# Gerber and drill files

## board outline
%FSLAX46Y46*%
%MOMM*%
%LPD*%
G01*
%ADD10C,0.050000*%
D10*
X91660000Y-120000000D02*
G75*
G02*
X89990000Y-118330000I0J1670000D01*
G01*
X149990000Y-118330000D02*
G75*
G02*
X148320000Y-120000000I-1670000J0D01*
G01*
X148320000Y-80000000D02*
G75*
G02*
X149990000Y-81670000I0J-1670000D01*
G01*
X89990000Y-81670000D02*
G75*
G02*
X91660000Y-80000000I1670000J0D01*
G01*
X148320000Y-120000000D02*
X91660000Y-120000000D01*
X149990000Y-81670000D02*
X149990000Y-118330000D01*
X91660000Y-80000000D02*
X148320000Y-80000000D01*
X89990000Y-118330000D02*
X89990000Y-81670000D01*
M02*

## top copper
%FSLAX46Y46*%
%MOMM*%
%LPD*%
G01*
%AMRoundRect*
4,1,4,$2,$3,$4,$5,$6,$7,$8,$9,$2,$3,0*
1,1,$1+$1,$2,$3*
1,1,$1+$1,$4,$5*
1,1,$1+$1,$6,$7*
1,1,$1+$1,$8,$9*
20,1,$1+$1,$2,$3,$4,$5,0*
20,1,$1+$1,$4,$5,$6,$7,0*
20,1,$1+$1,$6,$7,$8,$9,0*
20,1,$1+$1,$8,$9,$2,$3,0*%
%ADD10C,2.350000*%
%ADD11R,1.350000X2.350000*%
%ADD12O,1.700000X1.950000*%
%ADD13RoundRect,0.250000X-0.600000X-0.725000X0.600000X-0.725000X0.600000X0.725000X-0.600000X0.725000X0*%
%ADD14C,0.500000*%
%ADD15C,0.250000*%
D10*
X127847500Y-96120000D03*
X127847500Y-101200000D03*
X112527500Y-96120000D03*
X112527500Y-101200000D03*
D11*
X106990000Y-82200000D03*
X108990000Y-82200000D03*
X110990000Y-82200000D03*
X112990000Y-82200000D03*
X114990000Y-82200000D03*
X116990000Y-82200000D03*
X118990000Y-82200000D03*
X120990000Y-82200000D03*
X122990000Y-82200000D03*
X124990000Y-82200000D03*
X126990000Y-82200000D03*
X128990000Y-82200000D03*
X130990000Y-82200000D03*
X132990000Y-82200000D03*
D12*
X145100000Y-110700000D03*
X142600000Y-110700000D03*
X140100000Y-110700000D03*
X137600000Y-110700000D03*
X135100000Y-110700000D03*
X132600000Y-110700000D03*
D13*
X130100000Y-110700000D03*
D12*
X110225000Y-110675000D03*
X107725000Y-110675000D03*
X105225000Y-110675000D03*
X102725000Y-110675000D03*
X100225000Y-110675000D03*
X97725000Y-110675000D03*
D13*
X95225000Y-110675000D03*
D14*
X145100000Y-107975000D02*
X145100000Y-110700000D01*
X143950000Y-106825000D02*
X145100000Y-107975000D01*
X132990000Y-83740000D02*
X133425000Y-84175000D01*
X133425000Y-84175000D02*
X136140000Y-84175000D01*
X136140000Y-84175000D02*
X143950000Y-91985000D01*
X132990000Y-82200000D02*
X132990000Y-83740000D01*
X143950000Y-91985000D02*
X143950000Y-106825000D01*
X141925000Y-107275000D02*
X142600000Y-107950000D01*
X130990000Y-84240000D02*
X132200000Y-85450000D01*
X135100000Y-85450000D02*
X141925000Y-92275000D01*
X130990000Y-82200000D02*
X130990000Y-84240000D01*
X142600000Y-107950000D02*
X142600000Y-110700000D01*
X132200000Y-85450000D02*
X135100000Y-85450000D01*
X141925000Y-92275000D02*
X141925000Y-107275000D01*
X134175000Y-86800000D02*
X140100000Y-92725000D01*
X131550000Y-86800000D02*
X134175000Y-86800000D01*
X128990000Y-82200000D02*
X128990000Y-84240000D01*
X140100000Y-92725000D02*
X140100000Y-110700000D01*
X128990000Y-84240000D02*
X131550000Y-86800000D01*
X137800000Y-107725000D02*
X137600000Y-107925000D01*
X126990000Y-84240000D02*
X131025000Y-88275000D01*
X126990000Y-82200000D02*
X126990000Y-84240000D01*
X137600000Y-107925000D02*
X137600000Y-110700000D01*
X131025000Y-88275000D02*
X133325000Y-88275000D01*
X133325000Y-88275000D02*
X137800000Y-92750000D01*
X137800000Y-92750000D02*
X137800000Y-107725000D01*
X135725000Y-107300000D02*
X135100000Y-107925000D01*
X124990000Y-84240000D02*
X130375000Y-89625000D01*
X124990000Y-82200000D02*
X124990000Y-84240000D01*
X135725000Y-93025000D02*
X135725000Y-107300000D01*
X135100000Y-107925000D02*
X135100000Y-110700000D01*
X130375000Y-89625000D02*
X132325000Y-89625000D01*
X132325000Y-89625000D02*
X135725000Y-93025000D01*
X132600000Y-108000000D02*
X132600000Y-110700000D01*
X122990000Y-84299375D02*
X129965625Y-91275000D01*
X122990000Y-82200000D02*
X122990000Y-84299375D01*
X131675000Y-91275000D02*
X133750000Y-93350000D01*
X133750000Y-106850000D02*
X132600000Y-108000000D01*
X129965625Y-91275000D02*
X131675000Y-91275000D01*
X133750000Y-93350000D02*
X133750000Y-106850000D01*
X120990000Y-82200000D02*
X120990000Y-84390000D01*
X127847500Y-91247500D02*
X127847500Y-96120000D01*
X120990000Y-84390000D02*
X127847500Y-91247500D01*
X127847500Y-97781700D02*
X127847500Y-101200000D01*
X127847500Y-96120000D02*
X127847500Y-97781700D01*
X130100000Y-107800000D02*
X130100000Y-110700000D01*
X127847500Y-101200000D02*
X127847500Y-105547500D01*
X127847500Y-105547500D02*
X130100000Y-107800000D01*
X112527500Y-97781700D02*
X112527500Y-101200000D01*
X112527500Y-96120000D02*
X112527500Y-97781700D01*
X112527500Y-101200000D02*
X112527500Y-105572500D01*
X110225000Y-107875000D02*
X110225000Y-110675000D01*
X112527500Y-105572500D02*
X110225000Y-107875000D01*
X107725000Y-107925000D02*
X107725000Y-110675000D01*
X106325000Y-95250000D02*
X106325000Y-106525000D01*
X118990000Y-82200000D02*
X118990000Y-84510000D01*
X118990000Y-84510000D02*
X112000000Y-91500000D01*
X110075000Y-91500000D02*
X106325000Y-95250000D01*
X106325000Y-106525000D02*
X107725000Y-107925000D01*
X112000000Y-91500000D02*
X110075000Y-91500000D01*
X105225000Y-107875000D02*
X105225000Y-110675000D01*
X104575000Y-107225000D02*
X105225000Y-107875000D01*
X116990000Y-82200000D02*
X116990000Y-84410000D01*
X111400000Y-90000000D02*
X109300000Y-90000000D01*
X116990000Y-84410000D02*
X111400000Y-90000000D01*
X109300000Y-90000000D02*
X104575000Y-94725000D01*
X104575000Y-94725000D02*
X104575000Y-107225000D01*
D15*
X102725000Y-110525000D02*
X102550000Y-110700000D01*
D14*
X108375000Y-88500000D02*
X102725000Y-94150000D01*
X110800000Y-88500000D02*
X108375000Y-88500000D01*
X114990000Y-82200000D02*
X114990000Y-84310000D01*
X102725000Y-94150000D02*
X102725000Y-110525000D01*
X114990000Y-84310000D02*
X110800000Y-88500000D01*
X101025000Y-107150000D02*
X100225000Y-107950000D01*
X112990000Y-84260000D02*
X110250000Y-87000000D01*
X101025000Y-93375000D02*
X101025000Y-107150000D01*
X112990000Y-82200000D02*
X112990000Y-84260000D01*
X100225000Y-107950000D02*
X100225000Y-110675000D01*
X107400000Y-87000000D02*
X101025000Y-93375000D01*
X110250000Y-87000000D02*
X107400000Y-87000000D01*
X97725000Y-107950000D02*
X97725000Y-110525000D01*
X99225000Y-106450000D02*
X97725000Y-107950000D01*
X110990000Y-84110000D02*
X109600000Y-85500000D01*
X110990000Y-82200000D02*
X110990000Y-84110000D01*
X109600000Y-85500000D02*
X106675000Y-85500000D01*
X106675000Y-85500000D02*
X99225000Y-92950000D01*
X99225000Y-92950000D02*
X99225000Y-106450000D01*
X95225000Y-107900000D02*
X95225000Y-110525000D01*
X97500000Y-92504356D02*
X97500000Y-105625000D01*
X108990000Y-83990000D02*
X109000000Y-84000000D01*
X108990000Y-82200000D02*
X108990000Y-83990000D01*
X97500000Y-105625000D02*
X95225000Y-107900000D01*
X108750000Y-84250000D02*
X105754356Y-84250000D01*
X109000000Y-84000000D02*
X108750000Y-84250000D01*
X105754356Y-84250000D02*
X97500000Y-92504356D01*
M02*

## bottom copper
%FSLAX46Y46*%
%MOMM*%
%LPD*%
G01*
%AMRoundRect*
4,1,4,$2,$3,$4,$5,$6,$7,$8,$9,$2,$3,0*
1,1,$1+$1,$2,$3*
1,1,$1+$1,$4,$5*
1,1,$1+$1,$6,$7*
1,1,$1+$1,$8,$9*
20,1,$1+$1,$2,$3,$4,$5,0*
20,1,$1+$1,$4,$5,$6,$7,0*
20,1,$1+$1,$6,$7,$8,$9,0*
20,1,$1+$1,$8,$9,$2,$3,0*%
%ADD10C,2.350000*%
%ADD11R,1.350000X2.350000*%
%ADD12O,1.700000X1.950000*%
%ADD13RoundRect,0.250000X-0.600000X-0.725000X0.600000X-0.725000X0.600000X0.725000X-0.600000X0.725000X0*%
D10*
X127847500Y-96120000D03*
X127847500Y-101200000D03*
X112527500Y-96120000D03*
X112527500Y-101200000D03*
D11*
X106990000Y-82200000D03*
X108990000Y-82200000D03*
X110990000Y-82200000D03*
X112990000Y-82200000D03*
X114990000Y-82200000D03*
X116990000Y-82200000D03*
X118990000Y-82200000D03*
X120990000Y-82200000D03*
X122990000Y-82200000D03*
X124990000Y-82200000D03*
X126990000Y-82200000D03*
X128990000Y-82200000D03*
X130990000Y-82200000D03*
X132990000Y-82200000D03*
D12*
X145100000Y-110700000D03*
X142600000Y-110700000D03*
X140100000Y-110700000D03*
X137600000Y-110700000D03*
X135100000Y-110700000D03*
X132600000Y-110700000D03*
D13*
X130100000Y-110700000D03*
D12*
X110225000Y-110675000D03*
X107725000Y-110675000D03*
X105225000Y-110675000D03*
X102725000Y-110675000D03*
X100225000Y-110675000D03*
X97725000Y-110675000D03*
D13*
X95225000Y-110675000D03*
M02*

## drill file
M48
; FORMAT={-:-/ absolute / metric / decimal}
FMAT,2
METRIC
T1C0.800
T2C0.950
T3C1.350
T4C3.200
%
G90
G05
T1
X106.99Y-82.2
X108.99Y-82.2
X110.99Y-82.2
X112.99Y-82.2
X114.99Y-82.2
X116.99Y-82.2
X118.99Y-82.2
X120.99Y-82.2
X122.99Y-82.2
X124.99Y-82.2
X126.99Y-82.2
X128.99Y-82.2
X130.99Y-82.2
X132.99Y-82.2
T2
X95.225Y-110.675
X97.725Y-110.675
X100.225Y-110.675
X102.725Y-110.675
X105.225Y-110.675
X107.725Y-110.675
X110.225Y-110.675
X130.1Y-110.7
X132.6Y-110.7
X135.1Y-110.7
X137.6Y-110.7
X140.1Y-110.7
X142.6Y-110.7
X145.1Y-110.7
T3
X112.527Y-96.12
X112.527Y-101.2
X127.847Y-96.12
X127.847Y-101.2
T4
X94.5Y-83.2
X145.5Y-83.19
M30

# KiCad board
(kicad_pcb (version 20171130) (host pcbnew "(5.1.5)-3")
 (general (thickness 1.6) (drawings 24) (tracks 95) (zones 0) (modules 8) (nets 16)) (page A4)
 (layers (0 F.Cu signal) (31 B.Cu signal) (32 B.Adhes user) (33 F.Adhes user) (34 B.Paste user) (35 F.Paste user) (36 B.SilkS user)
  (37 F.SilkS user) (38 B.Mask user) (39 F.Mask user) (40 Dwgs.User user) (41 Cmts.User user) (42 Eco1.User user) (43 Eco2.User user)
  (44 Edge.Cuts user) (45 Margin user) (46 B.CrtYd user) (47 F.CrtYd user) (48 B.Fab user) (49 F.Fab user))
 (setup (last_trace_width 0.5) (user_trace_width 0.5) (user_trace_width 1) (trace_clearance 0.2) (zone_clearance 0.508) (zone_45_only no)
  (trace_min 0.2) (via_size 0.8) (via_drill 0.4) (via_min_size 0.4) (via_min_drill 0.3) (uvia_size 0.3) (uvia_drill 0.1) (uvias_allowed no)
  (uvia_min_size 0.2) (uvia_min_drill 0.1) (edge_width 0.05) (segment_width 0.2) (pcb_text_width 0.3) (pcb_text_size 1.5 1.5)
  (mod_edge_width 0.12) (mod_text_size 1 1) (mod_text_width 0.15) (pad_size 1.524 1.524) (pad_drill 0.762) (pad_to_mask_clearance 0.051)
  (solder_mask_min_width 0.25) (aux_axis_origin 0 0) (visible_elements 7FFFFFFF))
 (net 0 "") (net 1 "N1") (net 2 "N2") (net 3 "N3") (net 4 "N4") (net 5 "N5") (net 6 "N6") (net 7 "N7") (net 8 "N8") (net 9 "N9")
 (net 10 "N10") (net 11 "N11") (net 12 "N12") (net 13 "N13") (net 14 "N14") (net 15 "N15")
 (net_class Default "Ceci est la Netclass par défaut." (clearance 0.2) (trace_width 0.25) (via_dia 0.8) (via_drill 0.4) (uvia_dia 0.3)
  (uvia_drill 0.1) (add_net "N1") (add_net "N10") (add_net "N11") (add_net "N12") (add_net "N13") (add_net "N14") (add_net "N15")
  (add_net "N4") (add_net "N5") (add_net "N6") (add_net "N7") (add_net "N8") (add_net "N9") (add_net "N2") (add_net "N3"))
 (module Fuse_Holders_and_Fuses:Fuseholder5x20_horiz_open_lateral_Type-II (layer F.Cu) (at 127.8475 101.2 180)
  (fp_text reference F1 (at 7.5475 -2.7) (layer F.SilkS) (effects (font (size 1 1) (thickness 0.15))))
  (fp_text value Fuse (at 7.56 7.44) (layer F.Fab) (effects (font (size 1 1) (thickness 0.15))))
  (pad 1 thru_hole circle (at 0 5.08 180) (size 2.35 2.35) (drill 1.35) (layers *.Cu *.Mask) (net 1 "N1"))
  (pad 1 thru_hole circle (at 0 0 180) (size 2.35 2.35) (drill 1.35) (layers *.Cu *.Mask) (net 1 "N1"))
  (pad 2 thru_hole circle (at 15.32 5.08 180) (size 2.35 2.35) (drill 1.35) (layers *.Cu *.Mask) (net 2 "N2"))
  (pad 2 thru_hole circle (at 15.32 0 180) (size 2.35 2.35) (drill 1.35) (layers *.Cu *.Mask) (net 2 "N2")))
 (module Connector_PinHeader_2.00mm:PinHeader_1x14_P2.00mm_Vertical (layer B.Cu) (at 132.99 82.2 90)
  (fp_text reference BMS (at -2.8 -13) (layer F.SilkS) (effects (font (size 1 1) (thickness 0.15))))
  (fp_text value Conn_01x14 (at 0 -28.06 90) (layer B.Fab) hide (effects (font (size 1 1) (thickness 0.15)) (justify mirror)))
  (pad 14 thru_hole rect (at 0 -26 90) (size 2.35 1.35) (drill 0.8) (layers *.Cu *.Mask) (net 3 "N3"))
  (pad 13 thru_hole rect (at 0 -24 90) (size 2.35 1.35) (drill 0.8) (layers *.Cu *.Mask) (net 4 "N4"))
  (pad 12 thru_hole rect (at 0 -22 90) (size 2.35 1.35) (drill 0.8) (layers *.Cu *.Mask) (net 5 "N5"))
  (pad 11 thru_hole rect (at 0 -20 90) (size 2.35 1.35) (drill 0.8) (layers *.Cu *.Mask) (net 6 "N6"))
  (pad 10 thru_hole rect (at 0 -18 90) (size 2.35 1.35) (drill 0.8) (layers *.Cu *.Mask) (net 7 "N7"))
  (pad 9 thru_hole rect (at 0 -16 90) (size 2.35 1.35) (drill 0.8) (layers *.Cu *.Mask) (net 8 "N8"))
  (pad 8 thru_hole rect (at 0 -14 90) (size 2.35 1.35) (drill 0.8) (layers *.Cu *.Mask) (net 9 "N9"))
  (pad 7 thru_hole rect (at 0 -12 90) (size 2.35 1.35) (drill 0.8) (layers *.Cu *.Mask) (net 1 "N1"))
  (pad 6 thru_hole rect (at 0 -10 90) (size 2.35 1.35) (drill 0.8) (layers *.Cu *.Mask) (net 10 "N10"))
  (pad 5 thru_hole rect (at 0 -8 90) (size 2.35 1.35) (drill 0.8) (layers *.Cu *.Mask) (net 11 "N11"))
  (pad 4 thru_hole rect (at 0 -6 90) (size 2.35 1.35) (drill 0.8) (layers *.Cu *.Mask) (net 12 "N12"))
  (pad 3 thru_hole rect (at 0 -4 90) (size 2.35 1.35) (drill 0.8) (layers *.Cu *.Mask) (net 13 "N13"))
  (pad 2 thru_hole rect (at 0 -2 90) (size 2.35 1.35) (drill 0.8) (layers *.Cu *.Mask) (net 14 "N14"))
  (pad 1 thru_hole rect (at 0 0 90) (size 2.35 1.35) (drill 0.8) (layers *.Cu *.Mask) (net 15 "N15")))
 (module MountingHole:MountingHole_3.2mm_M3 (layer F.Cu) (at 145.5 83.19)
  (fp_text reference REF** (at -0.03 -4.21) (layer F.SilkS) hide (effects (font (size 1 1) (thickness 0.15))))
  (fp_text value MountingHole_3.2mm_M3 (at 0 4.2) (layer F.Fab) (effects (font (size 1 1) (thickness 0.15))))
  (pad 1 np_thru_hole circle (at 0 0) (size 3.2 3.2) (drill 3.2) (layers *.Cu *.Mask)))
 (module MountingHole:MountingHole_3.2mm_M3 (layer F.Cu) (at 94.5 83.2)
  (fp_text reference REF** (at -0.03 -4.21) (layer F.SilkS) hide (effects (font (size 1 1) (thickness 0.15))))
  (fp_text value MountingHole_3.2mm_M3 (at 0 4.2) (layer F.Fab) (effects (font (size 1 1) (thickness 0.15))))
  (pad 1 np_thru_hole circle (at 0 0) (size 3.2 3.2) (drill 3.2) (layers *.Cu *.Mask)))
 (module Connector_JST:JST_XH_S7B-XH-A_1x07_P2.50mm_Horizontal (layer F.Cu) (at 130.1 110.7)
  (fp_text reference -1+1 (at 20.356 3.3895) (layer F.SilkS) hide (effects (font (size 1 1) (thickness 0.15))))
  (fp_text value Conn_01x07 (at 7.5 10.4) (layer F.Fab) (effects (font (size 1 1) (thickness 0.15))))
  (pad 7 thru_hole oval (at 15 0) (size 1.7 1.95) (drill 0.95) (layers *.Cu *.Mask) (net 15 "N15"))
  (pad 6 thru_hole oval (at 12.5 0) (size 1.7 1.95) (drill 0.95) (layers *.Cu *.Mask) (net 14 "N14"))
  (pad 5 thru_hole oval (at 10 0) (size 1.7 1.95) (drill 0.95) (layers *.Cu *.Mask) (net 13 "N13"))
  (pad 4 thru_hole oval (at 7.5 0) (size 1.7 1.95) (drill 0.95) (layers *.Cu *.Mask) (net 12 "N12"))
  (pad 3 thru_hole oval (at 5 0) (size 1.7 1.95) (drill 0.95) (layers *.Cu *.Mask) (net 11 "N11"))
  (pad 2 thru_hole oval (at 2.5 0) (size 1.7 1.95) (drill 0.95) (layers *.Cu *.Mask) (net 10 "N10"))
  (pad 1 thru_hole roundrect (at 0 0) (size 1.7 1.95) (drill 0.95) (layers *.Cu *.Mask) (roundrect_rratio 0.147059) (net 1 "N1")))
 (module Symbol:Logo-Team (layer F.Cu) (at 97 92.59)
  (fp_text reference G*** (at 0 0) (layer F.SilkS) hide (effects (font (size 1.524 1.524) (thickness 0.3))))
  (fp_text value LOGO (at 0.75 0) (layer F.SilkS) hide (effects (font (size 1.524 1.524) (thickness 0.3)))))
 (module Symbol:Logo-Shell (layer F.Cu) (at 142.57 91.74)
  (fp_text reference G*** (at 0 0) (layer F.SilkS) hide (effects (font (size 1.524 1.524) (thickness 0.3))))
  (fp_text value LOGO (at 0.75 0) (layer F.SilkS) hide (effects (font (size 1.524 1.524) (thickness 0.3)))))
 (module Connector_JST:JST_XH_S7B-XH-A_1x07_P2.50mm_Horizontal (layer F.Cu) (at 95.225 110.675)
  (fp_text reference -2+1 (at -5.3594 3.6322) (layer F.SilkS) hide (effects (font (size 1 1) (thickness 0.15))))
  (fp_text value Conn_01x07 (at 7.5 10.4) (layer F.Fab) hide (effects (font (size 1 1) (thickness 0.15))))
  (pad 7 thru_hole oval (at 15 0) (size 1.7 1.95) (drill 0.95) (layers *.Cu *.Mask) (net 2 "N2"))
  (pad 6 thru_hole oval (at 12.5 0) (size 1.7 1.95) (drill 0.95) (layers *.Cu *.Mask) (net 9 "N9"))
  (pad 5 thru_hole oval (at 10 0) (size 1.7 1.95) (drill 0.95) (layers *.Cu *.Mask) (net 8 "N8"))
  (pad 4 thru_hole oval (at 7.5 0) (size 1.7 1.95) (drill 0.95) (layers *.Cu *.Mask) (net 7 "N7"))
  (pad 3 thru_hole oval (at 5 0) (size 1.7 1.95) (drill 0.95) (layers *.Cu *.Mask) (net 6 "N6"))
  (pad 2 thru_hole oval (at 2.5 0) (size 1.7 1.95) (drill 0.95) (layers *.Cu *.Mask) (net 5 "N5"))
  (pad 1 thru_hole roundrect (at 0 0) (size 1.7 1.95) (drill 0.95) (layers *.Cu *.Mask) (roundrect_rratio 0.147059) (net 4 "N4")))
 (gr_arc (start 91.66 118.33) (end 89.99 118.33) (angle -90) (layer Edge.Cuts) (width 0.05))
 (gr_arc (start 148.32 118.33) (end 148.32 120) (angle -90) (layer Edge.Cuts) (width 0.05))
 (gr_arc (start 148.32 81.67) (end 149.99 81.67) (angle -90) (layer Edge.Cuts) (width 0.05))
 (gr_arc (start 91.66 81.67) (end 91.66 80) (angle -90) (layer Edge.Cuts) (width 0.05))
 (gr_line (start 148.32 120) (end 91.66 120) (layer Edge.Cuts) (width 0.05))
 (gr_line (start 149.99 81.67) (end 149.99 118.33) (layer Edge.Cuts) (width 0.05))
 (gr_line (start 91.66 80) (end 148.32 80) (layer Edge.Cuts) (width 0.05))
 (gr_line (start 89.99 118.33) (end 89.99 81.67) (layer Edge.Cuts) (width 0.05))
 (segment (start 145.1 107.975) (end 145.1 110.7) (width 0.5) (layer F.Cu) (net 15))
 (segment (start 143.95 106.825) (end 145.1 107.975) (width 0.5) (layer F.Cu) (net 15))
 (segment (start 132.99 83.74) (end 133.425 84.175) (width 0.5) (layer F.Cu) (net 15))
 (segment (start 133.425 84.175) (end 136.14 84.175) (width 0.5) (layer F.Cu) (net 15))
 (segment (start 136.14 84.175) (end 143.95 91.985) (width 0.5) (layer F.Cu) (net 15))
 (segment (start 132.99 82.2) (end 132.99 83.74) (width 0.5) (layer F.Cu) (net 15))
 (segment (start 143.95 91.985) (end 143.95 106.825) (width 0.5) (layer F.Cu) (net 15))
 (segment (start 141.925 107.275) (end 142.6 107.95) (width 0.5) (layer F.Cu) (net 14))
 (segment (start 130.99 84.24) (end 132.2 85.45) (width 0.5) (layer F.Cu) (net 14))
 (segment (start 135.1 85.45) (end 141.925 92.275) (width 0.5) (layer F.Cu) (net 14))
 (segment (start 130.99 82.2) (end 130.99 84.24) (width 0.5) (layer F.Cu) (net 14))
 (segment (start 142.6 107.95) (end 142.6 110.7) (width 0.5) (layer F.Cu) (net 14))
 (segment (start 132.2 85.45) (end 135.1 85.45) (width 0.5) (layer F.Cu) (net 14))
 (segment (start 141.925 92.275) (end 141.925 107.275) (width 0.5) (layer F.Cu) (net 14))
 (segment (start 134.175 86.8) (end 140.1 92.725) (width 0.5) (layer F.Cu) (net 13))
 (segment (start 131.55 86.8) (end 134.175 86.8) (width 0.5) (layer F.Cu) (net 13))
 (segment (start 128.99 82.2) (end 128.99 84.24) (width 0.5) (layer F.Cu) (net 13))
 (segment (start 140.1 92.725) (end 140.1 110.7) (width 0.5) (layer F.Cu) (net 13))
 (segment (start 128.99 84.24) (end 131.55 86.8) (width 0.5) (layer F.Cu) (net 13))
 (segment (start 137.8 107.725) (end 137.6 107.925) (width 0.5) (layer F.Cu) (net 12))
 (segment (start 126.99 84.24) (end 131.025 88.275) (width 0.5) (layer F.Cu) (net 12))
 (segment (start 126.99 82.2) (end 126.99 84.24) (width 0.5) (layer F.Cu) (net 12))
 (segment (start 137.6 107.925) (end 137.6 110.7) (width 0.5) (layer F.Cu) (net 12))
 (segment (start 131.025 88.275) (end 133.325 88.275) (width 0.5) (layer F.Cu) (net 12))
 (segment (start 133.325 88.275) (end 137.8 92.75) (width 0.5) (layer F.Cu) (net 12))
 (segment (start 137.8 92.75) (end 137.8 107.725) (width 0.5) (layer F.Cu) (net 12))
 (segment (start 135.725 107.3) (end 135.1 107.925) (width 0.5) (layer F.Cu) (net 11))
 (segment (start 124.99 84.24) (end 130.375 89.625) (width 0.5) (layer F.Cu) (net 11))
 (segment (start 124.99 82.2) (end 124.99 84.24) (width 0.5) (layer F.Cu) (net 11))
 (segment (start 135.725 93.025) (end 135.725 107.3) (width 0.5) (layer F.Cu) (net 11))
 (segment (start 135.1 107.925) (end 135.1 110.7) (width 0.5) (layer F.Cu) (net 11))
 (segment (start 130.375 89.625) (end 132.325 89.625) (width 0.5) (layer F.Cu) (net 11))
 (segment (start 132.325 89.625) (end 135.725 93.025) (width 0.5) (layer F.Cu) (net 11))
 (segment (start 132.6 108) (end 132.6 110.7) (width 0.5) (layer F.Cu) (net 10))
 (segment (start 122.99 84.299375) (end 129.965625 91.275) (width 0.5) (layer F.Cu) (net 10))
 (segment (start 122.99 82.2) (end 122.99 84.299375) (width 0.5) (layer F.Cu) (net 10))
 (segment (start 131.675 91.275) (end 133.75 93.35) (width 0.5) (layer F.Cu) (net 10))
 (segment (start 133.75 106.85) (end 132.6 108) (width 0.5) (layer F.Cu) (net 10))
 (segment (start 129.965625 91.275) (end 131.675 91.275) (width 0.5) (layer F.Cu) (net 10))
 (segment (start 133.75 93.35) (end 133.75 106.85) (width 0.5) (layer F.Cu) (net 10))
 (segment (start 120.99 82.2) (end 120.99 84.39) (width 0.5) (layer F.Cu) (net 1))
 (segment (start 127.8475 91.2475) (end 127.8475 96.12) (width 0.5) (layer F.Cu) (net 1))
 (segment (start 120.99 84.39) (end 127.8475 91.2475) (width 0.5) (layer F.Cu) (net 1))
 (segment (start 127.8475 97.7817) (end 127.8475 101.2) (width 0.5) (layer F.Cu) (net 1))
 (segment (start 127.8475 96.12) (end 127.8475 97.7817) (width 0.5) (layer F.Cu) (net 1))
 (segment (start 130.1 107.8) (end 130.1 110.7) (width 0.5) (layer F.Cu) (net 1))
 (segment (start 127.8475 101.2) (end 127.8475 105.5475) (width 0.5) (layer F.Cu) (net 1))
 (segment (start 127.8475 105.5475) (end 130.1 107.8) (width 0.5) (layer F.Cu) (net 1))
 (segment (start 112.5275 97.7817) (end 112.5275 101.2) (width 0.5) (layer F.Cu) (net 2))
 (segment (start 112.5275 96.12) (end 112.5275 97.7817) (width 0.5) (layer F.Cu) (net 2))
 (segment (start 112.5275 101.2) (end 112.5275 105.5725) (width 0.5) (layer F.Cu) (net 2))
 (segment (start 110.225 107.875) (end 110.225 110.675) (width 0.5) (layer F.Cu) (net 2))
 (segment (start 112.5275 105.5725) (end 110.225 107.875) (width 0.5) (layer F.Cu) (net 2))
 (segment (start 107.725 107.925) (end 107.725 110.675) (width 0.5) (layer F.Cu) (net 9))
 (segment (start 106.325 95.25) (end 106.325 106.525) (width 0.5) (layer F.Cu) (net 9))
 (segment (start 118.99 82.2) (end 118.99 84.51) (width 0.5) (layer F.Cu) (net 9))
 (segment (start 118.99 84.51) (end 112 91.5) (width 0.5) (layer F.Cu) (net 9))
 (segment (start 110.075 91.5) (end 106.325 95.25) (width 0.5) (layer F.Cu) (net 9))
 (segment (start 106.325 106.525) (end 107.725 107.925) (width 0.5) (layer F.Cu) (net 9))
 (segment (start 112 91.5) (end 110.075 91.5) (width 0.5) (layer F.Cu) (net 9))
 (segment (start 105.225 107.875) (end 105.225 110.675) (width 0.5) (layer F.Cu) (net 8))
 (segment (start 104.575 107.225) (end 105.225 107.875) (width 0.5) (layer F.Cu) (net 8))
 (segment (start 116.99 82.2) (end 116.99 84.41) (width 0.5) (layer F.Cu) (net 8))
 (segment (start 111.4 90) (end 109.3 90) (width 0.5) (layer F.Cu) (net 8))
 (segment (start 116.99 84.41) (end 111.4 90) (width 0.5) (layer F.Cu) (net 8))
 (segment (start 109.3 90) (end 104.575 94.725) (width 0.5) (layer F.Cu) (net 8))
 (segment (start 104.575 94.725) (end 104.575 107.225) (width 0.5) (layer F.Cu) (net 8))
 (segment (start 102.725 110.525) (end 102.55 110.7) (width 0.25) (layer F.Cu) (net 7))
 (segment (start 108.375 88.5) (end 102.725 94.15) (width 0.5) (layer F.Cu) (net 7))
 (segment (start 110.8 88.5) (end 108.375 88.5) (width 0.5) (layer F.Cu) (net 7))
 (segment (start 114.99 82.2) (end 114.99 84.31) (width 0.5) (layer F.Cu) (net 7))
 (segment (start 102.725 94.15) (end 102.725 110.525) (width 0.5) (layer F.Cu) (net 7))
 (segment (start 114.99 84.31) (end 110.8 88.5) (width 0.5) (layer F.Cu) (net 7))
 (segment (start 101.025 107.15) (end 100.225 107.95) (width 0.5) (layer F.Cu) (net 6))
 (segment (start 112.99 84.26) (end 110.25 87) (width 0.5) (layer F.Cu) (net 6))
 (segment (start 101.025 93.375) (end 101.025 107.15) (width 0.5) (layer F.Cu) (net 6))
 (segment (start 112.99 82.2) (end 112.99 84.26) (width 0.5) (layer F.Cu) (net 6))
 (segment (start 100.225 107.95) (end 100.225 110.675) (width 0.5) (layer F.Cu) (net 6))
 (segment (start 107.4 87) (end 101.025 93.375) (width 0.5) (layer F.Cu) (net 6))
 (segment (start 110.25 87) (end 107.4 87) (width 0.5) (layer F.Cu) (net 6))
 (segment (start 97.725 107.95) (end 97.725 110.525) (width 0.5) (layer F.Cu) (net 5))
 (segment (start 99.225 106.45) (end 97.725 107.95) (width 0.5) (layer F.Cu) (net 5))
 (segment (start 110.99 84.11) (end 109.6 85.5) (width 0.5) (layer F.Cu) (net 5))
 (segment (start 110.99 82.2) (end 110.99 84.11) (width 0.5) (layer F.Cu) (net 5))
 (segment (start 109.6 85.5) (end 106.675 85.5) (width 0.5) (layer F.Cu) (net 5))
 (segment (start 106.675 85.5) (end 99.225 92.95) (width 0.5) (layer F.Cu) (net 5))
 (segment (start 99.225 92.95) (end 99.225 106.45) (width 0.5) (layer F.Cu) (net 5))
 (segment (start 95.225 107.9) (end 95.225 110.525) (width 0.5) (layer F.Cu) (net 4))
 (segment (start 97.5 92.504356) (end 97.5 105.625) (width 0.5) (layer F.Cu) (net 4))
 (segment (start 108.99 83.99) (end 109 84) (width 0.5) (layer F.Cu) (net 4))
 (segment (start 108.99 82.2) (end 108.99 83.99) (width 0.5) (layer F.Cu) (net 4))
 (segment (start 97.5 105.625) (end 95.225 107.9) (width 0.5) (layer F.Cu) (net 4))
 (segment (start 108.75 84.25) (end 105.754356 84.25) (width 0.5) (layer F.Cu) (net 4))
 (segment (start 109 84) (end 108.75 84.25) (width 0.5) (layer F.Cu) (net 4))
 (segment (start 105.754356 84.25) (end 97.5 92.504356) (width 0.5) (layer F.Cu) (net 4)))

